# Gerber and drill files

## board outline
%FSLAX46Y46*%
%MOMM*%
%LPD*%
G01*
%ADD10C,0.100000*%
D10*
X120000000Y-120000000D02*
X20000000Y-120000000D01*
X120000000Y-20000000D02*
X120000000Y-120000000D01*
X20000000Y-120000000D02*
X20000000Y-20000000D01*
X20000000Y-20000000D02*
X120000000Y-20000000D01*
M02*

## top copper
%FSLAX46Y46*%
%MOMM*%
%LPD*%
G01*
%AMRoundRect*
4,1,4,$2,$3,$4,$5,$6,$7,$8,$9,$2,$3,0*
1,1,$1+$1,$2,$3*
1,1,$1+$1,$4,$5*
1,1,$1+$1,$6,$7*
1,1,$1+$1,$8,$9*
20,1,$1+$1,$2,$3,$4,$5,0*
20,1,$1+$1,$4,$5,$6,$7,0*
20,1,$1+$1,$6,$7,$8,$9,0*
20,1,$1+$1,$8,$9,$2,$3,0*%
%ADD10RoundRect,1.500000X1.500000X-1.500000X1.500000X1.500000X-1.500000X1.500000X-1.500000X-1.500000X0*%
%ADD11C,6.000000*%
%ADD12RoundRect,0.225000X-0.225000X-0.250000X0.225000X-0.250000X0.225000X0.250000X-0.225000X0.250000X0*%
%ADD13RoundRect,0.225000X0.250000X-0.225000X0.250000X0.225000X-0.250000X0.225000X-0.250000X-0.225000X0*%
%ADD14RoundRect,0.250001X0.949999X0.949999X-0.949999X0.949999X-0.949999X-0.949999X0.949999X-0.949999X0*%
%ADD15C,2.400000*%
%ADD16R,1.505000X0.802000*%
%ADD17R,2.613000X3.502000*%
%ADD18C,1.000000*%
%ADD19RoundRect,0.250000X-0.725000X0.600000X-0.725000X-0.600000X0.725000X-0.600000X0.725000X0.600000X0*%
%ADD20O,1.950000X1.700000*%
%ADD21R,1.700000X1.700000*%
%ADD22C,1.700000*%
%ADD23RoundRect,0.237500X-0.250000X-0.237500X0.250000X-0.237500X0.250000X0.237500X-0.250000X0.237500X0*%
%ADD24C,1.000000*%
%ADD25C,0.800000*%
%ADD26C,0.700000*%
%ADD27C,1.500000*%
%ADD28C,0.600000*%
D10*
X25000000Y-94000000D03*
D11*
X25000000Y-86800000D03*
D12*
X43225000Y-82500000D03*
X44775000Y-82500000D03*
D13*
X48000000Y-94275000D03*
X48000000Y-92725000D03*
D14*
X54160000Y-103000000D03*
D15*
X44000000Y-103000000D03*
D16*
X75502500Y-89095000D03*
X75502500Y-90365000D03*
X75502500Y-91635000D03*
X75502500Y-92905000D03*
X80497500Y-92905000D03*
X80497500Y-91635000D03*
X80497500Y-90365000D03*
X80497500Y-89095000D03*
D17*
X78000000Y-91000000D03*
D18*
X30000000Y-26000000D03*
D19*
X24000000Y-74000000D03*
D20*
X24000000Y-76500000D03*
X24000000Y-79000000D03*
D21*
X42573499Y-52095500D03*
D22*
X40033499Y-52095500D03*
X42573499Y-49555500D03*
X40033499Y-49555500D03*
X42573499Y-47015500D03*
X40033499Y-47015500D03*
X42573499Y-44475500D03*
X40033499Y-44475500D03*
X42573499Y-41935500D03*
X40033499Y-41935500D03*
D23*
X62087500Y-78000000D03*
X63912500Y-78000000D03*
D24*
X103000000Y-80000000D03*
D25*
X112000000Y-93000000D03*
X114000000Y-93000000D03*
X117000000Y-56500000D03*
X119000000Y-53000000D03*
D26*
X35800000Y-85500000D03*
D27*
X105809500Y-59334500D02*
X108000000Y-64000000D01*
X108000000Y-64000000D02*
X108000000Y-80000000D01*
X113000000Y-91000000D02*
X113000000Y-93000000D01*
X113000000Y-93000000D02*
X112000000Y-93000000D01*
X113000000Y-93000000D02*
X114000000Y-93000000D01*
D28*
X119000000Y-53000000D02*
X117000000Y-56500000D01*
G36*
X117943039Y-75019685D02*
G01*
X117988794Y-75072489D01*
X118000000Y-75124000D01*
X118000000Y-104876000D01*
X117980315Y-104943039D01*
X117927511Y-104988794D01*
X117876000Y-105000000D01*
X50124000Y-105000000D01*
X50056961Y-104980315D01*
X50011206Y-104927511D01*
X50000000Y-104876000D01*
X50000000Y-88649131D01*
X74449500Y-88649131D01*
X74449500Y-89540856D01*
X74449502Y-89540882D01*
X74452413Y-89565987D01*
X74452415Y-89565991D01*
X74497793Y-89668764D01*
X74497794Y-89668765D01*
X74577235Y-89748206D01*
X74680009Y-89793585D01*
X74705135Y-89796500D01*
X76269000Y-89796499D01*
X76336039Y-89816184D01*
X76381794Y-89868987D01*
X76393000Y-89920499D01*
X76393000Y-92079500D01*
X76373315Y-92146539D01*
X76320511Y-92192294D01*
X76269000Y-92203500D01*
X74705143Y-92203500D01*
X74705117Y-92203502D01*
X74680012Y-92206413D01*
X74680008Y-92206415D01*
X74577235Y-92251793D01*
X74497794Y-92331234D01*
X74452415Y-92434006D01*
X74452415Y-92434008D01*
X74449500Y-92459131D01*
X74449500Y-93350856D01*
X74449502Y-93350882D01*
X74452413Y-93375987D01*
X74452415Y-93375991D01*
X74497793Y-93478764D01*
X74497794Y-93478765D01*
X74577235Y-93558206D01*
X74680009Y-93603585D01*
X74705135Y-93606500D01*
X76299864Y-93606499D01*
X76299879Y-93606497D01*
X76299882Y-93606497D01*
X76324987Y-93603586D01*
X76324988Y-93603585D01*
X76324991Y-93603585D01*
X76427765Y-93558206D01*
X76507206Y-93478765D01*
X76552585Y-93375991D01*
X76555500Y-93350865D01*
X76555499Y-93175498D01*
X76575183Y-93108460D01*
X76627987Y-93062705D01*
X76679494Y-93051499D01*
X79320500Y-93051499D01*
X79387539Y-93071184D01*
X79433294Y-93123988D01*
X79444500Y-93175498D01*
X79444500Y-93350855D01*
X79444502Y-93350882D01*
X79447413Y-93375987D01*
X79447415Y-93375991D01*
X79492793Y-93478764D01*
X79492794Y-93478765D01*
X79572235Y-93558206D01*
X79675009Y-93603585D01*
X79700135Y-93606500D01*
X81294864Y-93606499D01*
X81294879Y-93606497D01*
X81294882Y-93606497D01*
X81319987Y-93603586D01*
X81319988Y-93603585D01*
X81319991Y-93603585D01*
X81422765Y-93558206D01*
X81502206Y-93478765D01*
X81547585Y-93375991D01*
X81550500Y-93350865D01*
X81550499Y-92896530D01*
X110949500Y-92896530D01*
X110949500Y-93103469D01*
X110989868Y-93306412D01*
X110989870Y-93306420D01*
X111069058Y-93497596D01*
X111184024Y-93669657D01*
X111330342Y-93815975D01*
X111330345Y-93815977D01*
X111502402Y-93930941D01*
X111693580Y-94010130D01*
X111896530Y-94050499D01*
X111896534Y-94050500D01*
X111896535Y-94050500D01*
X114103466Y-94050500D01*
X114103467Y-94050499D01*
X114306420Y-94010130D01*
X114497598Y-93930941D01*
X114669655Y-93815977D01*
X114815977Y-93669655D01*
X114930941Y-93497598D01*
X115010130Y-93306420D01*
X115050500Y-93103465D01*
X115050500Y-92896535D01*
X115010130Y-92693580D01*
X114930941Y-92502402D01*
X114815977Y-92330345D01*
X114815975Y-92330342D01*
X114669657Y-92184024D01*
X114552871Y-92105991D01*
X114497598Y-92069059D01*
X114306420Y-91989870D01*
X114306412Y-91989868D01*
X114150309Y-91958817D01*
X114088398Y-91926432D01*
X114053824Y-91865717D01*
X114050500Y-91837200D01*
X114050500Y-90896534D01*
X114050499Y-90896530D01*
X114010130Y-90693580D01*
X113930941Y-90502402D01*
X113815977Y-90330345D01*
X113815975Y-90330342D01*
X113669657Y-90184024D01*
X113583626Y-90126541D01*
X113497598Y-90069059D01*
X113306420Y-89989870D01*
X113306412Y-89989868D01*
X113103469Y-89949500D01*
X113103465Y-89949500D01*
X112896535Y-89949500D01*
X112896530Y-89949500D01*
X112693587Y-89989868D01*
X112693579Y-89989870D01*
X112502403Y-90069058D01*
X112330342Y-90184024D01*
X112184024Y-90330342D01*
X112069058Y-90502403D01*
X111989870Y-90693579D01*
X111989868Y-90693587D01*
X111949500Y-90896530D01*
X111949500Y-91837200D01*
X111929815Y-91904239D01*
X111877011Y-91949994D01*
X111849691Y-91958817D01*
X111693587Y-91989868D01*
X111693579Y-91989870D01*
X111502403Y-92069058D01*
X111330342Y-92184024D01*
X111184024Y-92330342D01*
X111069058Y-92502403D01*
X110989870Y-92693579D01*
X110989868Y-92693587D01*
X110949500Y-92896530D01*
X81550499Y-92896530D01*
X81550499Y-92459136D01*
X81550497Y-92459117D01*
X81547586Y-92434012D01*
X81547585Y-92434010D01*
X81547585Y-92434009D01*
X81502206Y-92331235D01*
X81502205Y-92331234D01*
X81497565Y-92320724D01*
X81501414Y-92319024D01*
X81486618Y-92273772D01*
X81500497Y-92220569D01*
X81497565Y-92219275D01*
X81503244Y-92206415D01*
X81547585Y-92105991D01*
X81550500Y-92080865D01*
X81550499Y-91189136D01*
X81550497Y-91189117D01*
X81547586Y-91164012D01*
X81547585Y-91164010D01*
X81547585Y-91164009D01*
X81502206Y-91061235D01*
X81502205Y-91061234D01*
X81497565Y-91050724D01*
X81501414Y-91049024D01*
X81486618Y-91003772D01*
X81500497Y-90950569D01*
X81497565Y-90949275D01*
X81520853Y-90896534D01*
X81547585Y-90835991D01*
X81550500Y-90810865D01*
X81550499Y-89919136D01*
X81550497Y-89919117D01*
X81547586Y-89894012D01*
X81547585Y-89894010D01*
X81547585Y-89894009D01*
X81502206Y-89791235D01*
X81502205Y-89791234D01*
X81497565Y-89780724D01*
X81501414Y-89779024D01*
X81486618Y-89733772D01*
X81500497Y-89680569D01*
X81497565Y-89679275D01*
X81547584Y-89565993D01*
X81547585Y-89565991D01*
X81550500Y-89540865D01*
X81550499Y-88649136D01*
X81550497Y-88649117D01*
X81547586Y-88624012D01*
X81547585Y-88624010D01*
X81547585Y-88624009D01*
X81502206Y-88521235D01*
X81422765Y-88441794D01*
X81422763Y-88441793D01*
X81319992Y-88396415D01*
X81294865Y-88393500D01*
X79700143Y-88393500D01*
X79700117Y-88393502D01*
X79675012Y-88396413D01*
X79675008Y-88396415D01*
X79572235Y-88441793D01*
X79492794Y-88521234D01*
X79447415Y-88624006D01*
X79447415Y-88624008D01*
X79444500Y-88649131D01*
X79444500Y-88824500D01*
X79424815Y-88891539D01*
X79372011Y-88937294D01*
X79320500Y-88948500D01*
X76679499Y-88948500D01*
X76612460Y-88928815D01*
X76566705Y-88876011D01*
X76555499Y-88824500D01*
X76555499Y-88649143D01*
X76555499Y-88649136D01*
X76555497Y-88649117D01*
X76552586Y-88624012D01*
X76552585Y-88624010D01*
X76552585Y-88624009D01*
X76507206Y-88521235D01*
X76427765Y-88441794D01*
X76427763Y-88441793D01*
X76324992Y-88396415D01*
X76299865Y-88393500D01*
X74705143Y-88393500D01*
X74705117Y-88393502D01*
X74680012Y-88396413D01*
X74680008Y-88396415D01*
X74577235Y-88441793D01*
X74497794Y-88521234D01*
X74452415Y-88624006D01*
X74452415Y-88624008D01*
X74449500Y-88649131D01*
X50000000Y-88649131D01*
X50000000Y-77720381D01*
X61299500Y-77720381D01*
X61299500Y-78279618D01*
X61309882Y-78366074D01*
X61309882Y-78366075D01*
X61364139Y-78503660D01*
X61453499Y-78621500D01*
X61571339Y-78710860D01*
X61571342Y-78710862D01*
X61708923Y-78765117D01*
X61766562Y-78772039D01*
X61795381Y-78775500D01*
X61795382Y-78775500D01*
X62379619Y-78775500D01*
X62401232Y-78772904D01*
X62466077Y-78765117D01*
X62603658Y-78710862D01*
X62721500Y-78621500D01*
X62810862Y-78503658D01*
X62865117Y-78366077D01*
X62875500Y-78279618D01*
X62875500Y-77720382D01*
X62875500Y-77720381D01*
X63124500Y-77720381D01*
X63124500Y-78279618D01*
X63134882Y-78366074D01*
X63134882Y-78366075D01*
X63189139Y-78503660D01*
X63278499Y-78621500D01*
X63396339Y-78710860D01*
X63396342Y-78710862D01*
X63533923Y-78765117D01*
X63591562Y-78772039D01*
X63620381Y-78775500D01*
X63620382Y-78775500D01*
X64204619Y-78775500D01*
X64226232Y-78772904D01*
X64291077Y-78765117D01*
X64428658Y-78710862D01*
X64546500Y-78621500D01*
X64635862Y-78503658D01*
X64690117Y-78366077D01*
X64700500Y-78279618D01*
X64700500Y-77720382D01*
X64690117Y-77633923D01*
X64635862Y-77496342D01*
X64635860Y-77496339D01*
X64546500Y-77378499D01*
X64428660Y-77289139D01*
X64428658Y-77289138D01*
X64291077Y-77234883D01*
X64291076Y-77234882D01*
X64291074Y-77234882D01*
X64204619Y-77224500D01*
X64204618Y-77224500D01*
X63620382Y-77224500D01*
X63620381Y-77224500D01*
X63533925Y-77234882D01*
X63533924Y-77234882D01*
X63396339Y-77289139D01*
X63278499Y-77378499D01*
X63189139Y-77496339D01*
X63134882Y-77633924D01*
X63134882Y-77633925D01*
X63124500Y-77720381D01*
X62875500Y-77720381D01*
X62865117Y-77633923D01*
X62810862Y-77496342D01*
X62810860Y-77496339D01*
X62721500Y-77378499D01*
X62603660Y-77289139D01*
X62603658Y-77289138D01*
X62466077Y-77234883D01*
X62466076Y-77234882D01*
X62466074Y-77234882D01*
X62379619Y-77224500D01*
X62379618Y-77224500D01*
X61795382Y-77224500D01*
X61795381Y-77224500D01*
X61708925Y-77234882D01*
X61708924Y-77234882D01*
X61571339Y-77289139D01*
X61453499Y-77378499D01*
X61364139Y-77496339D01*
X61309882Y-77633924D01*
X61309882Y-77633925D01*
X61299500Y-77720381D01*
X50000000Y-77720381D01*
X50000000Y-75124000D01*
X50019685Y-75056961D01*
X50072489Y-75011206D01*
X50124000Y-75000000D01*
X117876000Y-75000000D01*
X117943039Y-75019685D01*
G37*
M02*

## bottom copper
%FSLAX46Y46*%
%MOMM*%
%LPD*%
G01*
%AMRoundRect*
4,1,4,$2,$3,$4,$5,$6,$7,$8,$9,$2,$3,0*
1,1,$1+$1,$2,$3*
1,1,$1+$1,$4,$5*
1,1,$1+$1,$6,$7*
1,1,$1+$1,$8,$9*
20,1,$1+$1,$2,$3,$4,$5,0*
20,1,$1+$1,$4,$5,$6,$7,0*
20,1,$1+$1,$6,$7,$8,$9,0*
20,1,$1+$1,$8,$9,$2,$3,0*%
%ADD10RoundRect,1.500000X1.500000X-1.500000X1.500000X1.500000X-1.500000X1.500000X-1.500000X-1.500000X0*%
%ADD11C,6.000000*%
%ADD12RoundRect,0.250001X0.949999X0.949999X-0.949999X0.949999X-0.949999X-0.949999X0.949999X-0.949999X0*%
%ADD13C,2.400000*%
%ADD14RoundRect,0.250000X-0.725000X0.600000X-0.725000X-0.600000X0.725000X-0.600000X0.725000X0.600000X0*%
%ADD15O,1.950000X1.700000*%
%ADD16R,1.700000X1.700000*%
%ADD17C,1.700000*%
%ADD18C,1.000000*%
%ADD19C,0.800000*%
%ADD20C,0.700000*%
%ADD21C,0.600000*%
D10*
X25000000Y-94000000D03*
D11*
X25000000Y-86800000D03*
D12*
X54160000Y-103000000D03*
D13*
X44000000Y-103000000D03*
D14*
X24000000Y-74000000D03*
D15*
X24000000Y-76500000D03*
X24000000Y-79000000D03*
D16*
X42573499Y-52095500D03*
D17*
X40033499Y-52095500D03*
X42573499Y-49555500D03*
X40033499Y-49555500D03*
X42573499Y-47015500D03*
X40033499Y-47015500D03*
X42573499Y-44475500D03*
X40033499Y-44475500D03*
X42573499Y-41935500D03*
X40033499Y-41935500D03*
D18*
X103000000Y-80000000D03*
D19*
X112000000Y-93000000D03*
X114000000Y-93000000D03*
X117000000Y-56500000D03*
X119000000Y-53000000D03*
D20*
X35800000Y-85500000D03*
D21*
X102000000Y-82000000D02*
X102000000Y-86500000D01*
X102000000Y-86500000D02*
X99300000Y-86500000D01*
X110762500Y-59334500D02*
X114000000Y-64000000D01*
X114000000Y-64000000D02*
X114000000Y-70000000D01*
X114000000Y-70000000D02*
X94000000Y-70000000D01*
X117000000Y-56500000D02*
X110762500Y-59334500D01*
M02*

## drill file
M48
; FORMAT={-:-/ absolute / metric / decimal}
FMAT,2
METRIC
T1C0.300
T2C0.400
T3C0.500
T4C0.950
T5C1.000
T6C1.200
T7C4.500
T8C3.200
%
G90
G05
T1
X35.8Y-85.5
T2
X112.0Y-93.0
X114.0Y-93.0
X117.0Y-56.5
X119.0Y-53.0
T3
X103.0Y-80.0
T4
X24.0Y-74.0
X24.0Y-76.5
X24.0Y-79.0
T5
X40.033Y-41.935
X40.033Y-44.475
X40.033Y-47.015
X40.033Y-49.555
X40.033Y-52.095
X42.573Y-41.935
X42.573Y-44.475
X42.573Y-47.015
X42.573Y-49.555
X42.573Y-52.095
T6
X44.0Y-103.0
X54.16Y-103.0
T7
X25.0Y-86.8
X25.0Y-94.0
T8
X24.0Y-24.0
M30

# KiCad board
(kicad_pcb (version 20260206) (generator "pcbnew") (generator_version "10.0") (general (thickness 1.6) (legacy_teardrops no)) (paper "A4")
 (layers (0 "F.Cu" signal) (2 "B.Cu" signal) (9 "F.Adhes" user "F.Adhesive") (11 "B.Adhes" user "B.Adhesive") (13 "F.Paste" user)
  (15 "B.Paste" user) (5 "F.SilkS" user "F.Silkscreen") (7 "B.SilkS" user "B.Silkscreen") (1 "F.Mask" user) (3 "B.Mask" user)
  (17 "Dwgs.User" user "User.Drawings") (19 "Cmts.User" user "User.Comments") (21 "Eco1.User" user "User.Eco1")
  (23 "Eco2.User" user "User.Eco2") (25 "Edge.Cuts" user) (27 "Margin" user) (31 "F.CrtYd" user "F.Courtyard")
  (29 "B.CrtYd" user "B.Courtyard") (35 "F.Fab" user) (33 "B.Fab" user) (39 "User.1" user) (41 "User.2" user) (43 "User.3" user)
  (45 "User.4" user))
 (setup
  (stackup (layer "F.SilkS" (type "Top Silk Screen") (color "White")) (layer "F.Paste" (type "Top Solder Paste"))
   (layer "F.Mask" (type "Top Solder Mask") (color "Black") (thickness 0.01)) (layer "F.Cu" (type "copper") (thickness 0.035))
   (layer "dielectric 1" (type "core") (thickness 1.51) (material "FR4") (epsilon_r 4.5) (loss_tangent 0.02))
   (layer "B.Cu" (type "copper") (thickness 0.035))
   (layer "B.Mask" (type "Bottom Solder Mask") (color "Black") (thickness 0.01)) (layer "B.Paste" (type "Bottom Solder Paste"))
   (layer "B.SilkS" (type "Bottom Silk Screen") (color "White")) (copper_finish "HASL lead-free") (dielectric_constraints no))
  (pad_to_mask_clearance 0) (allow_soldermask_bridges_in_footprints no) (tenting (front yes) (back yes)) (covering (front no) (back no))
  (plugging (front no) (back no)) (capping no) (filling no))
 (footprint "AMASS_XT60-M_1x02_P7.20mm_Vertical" (layer "F.Cu") (at 25 94 90)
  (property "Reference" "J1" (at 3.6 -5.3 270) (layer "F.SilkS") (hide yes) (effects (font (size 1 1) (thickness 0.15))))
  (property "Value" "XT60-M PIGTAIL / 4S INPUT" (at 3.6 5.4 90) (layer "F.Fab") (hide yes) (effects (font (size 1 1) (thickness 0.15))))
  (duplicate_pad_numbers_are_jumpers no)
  (pad "1" thru_hole roundrect (at 0 0 90) (size 6 6) (drill 4.5) (layers "*.Cu" "*.Mask") (remove_unused_layers no) (roundrect_rratio 0.25)
   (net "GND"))
  (pad "2" thru_hole circle (at 7.2 0 90) (size 6 6) (drill 4.5) (layers "*.Cu" "*.Mask") (remove_unused_layers no) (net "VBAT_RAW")))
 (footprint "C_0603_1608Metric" (layer "F.Cu") (at 44 82.5)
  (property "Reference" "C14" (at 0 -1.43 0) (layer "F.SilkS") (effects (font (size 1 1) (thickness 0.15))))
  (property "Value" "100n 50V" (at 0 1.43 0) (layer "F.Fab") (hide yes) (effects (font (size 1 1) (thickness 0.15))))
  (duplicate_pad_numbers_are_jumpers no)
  (pad "1" smd roundrect (at -0.775 0) (size 0.9 0.95) (layers "F.Cu" "F.Mask" "F.Paste") (roundrect_rratio 0.25) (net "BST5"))
  (pad "2" smd roundrect (at 0.775 0) (size 0.9 0.95) (layers "F.Cu" "F.Mask" "F.Paste") (roundrect_rratio 0.25) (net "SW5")))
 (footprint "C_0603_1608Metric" (layer "F.Cu") (at 48 93.5 90)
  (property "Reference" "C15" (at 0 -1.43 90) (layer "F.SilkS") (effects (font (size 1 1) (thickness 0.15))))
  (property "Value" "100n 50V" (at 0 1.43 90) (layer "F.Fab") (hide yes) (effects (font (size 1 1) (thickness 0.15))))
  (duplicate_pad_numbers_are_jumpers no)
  (pad "1" smd roundrect (at -0.775 0 90) (size 0.9 0.95) (layers "F.Cu" "F.Mask" "F.Paste") (roundrect_rratio 0.25) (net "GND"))
  (pad "2" smd roundrect (at 0.775 0 90) (size 0.9 0.95) (layers "F.Cu" "F.Mask" "F.Paste") (roundrect_rratio 0.25) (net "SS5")))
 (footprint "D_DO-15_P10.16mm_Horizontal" (layer "F.Cu") (at 54.16 103 180)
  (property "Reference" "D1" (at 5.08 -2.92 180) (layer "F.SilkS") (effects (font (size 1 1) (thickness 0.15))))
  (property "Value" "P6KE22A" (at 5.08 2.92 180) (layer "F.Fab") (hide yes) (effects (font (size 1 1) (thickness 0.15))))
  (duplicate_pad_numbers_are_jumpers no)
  (pad "1" thru_hole roundrect (at 0 0 180) (size 2.4 2.4) (drill 1.2) (layers "*.Cu" "*.Mask") (remove_unused_layers no)
   (roundrect_rratio 0.104167) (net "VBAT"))
  (pad "2" thru_hole circle (at 10.16 0 180) (size 2.4 2.4) (drill 1.2) (layers "*.Cu" "*.Mask") (remove_unused_layers no) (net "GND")))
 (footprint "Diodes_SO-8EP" (layer "F.Cu") (at 78 91)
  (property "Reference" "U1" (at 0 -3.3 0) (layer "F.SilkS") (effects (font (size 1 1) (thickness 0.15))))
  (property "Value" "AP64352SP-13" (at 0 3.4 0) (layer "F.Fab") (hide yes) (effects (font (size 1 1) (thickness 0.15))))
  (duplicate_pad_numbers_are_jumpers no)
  (pad "1" smd rect (at -2.4975 -1.905) (size 1.505 0.802) (layers "F.Cu" "F.Mask" "F.Paste") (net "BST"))
  (pad "2" smd rect (at -2.4975 -0.635) (size 1.505 0.802) (layers "F.Cu" "F.Mask" "F.Paste") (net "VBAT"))
  (pad "3" smd rect (at -2.4975 0.635) (size 1.505 0.802) (layers "F.Cu" "F.Mask" "F.Paste") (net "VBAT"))
  (pad "4" smd rect (at -2.4975 1.905) (size 1.505 0.802) (layers "F.Cu" "F.Mask" "F.Paste") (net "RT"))
  (pad "5" smd rect (at 2.4975 1.905) (size 1.505 0.802) (layers "F.Cu" "F.Mask" "F.Paste") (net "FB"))
  (pad "6" smd rect (at 2.4975 0.635) (size 1.505 0.802) (layers "F.Cu" "F.Mask" "F.Paste") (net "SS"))
  (pad "7" smd rect (at 2.4975 -0.635) (size 1.505 0.802) (layers "F.Cu" "F.Mask" "F.Paste") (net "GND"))
  (pad "8" smd rect (at 2.4975 -1.905) (size 1.505 0.802) (layers "F.Cu" "F.Mask" "F.Paste") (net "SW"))
  (pad "9" smd rect (at 0 0) (size 2.613 3.502) (layers "F.Cu" "F.Mask" "F.Paste") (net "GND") (solder_paste_margin_ratio -0.2)))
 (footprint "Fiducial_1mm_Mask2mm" (layer "F.Cu") (at 30 26)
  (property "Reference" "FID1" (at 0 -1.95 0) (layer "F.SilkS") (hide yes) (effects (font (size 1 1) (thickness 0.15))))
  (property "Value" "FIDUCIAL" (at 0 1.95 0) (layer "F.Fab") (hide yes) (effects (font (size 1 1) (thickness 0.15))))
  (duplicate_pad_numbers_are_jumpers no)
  (pad "" smd circle (at 0 0) (size 1 1) (layers "F.Cu" "F.Mask") (solder_mask_margin 0.5) (clearance 0.6)))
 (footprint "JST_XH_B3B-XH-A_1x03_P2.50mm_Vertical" (layer "F.Cu") (at 24 74 -90)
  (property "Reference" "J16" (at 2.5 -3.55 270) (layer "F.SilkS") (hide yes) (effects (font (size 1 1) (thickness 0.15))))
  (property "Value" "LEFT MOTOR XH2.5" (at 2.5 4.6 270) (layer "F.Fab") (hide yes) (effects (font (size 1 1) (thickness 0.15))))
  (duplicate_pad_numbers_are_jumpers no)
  (pad "1" thru_hole roundrect (at 0 0 270) (size 1.7 1.95) (drill 0.95) (layers "*.Cu" "*.Mask") (remove_unused_layers no)
   (roundrect_rratio 0.147059) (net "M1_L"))
  (pad "2" thru_hole oval (at 2.5 0 270) (size 1.7 1.95) (drill 0.95) (layers "*.Cu" "*.Mask") (remove_unused_layers no) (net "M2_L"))
  (pad "3" thru_hole oval (at 5 0 270) (size 1.7 1.95) (drill 0.95) (layers "*.Cu" "*.Mask") (remove_unused_layers no) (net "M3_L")))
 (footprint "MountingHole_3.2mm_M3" (layer "F.Cu") (at 24 24)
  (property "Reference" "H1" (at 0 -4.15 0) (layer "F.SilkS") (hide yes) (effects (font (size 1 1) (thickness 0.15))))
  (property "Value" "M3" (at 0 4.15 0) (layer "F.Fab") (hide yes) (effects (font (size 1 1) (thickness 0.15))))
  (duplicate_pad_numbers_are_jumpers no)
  (pad "" np_thru_hole circle (at 0 0) (size 3.2 3.2) (drill 3.2) (layers "*.Cu" "*.Mask")))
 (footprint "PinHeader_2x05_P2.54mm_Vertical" (layer "F.Cu") (at 42.573499 52.0955 180)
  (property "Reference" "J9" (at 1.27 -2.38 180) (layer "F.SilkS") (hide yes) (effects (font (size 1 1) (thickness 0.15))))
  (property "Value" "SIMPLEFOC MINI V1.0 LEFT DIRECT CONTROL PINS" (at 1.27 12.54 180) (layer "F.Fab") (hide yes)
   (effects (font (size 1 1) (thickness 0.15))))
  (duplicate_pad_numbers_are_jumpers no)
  (pad "1" thru_hole rect (at 0 0 180) (size 1.7 1.7) (drill 1) (layers "*.Cu" "*.Mask") (remove_unused_layers no) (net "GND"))
  (pad "2" thru_hole circle (at 2.54 0 180) (size 1.7 1.7) (drill 1) (layers "*.Cu" "*.Mask") (remove_unused_layers no))
  (pad "3" thru_hole circle (at 0 2.54 180) (size 1.7 1.7) (drill 1) (layers "*.Cu" "*.Mask") (remove_unused_layers no) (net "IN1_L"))
  (pad "4" thru_hole circle (at 2.54 2.54 180) (size 1.7 1.7) (drill 1) (layers "*.Cu" "*.Mask") (remove_unused_layers no) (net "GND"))
  (pad "5" thru_hole circle (at 0 5.08 180) (size 1.7 1.7) (drill 1) (layers "*.Cu" "*.Mask") (remove_unused_layers no) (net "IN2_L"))
  (pad "6" thru_hole circle (at 2.54 5.08 180) (size 1.7 1.7) (drill 1) (layers "*.Cu" "*.Mask") (remove_unused_layers no))
  (pad "7" thru_hole circle (at 0 7.62 180) (size 1.7 1.7) (drill 1) (layers "*.Cu" "*.Mask") (remove_unused_layers no) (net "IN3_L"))
  (pad "8" thru_hole circle (at 2.54 7.62 180) (size 1.7 1.7) (drill 1) (layers "*.Cu" "*.Mask") (remove_unused_layers no))
  (pad "9" thru_hole circle (at 0 10.16 180) (size 1.7 1.7) (drill 1) (layers "*.Cu" "*.Mask") (remove_unused_layers no) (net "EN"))
  (pad "10" thru_hole circle (at 2.54 10.16 180) (size 1.7 1.7) (drill 1) (layers "*.Cu" "*.Mask") (remove_unused_layers no)
   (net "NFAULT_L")))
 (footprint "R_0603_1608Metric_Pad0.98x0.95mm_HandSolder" (layer "F.Cu") (at 63 78)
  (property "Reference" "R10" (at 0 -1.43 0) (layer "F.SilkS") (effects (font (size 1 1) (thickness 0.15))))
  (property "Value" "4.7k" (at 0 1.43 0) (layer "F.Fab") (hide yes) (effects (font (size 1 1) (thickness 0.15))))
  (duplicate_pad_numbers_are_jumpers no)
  (pad "1" smd roundrect (at -0.9125 0) (size 0.975 0.95) (layers "F.Cu" "F.Mask" "F.Paste") (roundrect_rratio 0.25) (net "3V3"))
  (pad "2" smd roundrect (at 0.9125 0) (size 0.975 0.95) (layers "F.Cu" "F.Mask" "F.Paste") (roundrect_rratio 0.25) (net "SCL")))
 (gr_line (start 120 120) (end 20 120) (stroke (width 0.1) (type default)) (layer "Edge.Cuts"))
 (gr_line (start 120 20) (end 120 120) (stroke (width 0.1) (type default)) (layer "Edge.Cuts"))
 (gr_line (start 20 120) (end 20 20) (stroke (width 0.1) (type default)) (layer "Edge.Cuts"))
 (gr_line (start 20 20) (end 120 20) (stroke (width 0.1) (type default)) (layer "Edge.Cuts"))
 (segment (start 102 82) (end 102 86.5) (width 0.6) (layer "B.Cu") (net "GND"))
 (segment (start 102 86.5) (end 99.3 86.5) (width 0.6) (layer "B.Cu") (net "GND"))
 (segment (start 105.8095 59.3345) (end 108 64) (width 1.5) (layer "F.Cu") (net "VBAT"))
 (segment (start 108 64) (end 108 80) (width 1.5) (layer "F.Cu") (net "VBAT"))
 (segment (start 110.7625 59.3345) (end 114 64) (width 0.6) (layer "B.Cu") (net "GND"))
 (segment (start 113 91) (end 113 93) (width 1.5) (layer "F.Cu") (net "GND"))
 (segment (start 113 93) (end 112 93) (width 1.5) (layer "F.Cu") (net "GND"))
 (segment (start 113 93) (end 114 93) (width 1.5) (layer "F.Cu") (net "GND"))
 (segment (start 114 64) (end 114 70) (width 0.6) (layer "B.Cu") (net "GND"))
 (segment (start 114 70) (end 94 70) (width 0.6) (layer "B.Cu") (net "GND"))
 (segment (start 117 56.5) (end 110.7625 59.3345) (width 0.6) (layer "B.Cu") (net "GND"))
 (segment (start 119 53) (end 117 56.5) (width 0.6) (layer "F.Cu") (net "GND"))
 (via (at 103 80) (size 1) (drill 0.5) (layers "F.Cu" "B.Cu") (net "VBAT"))
 (via (at 112 93) (size 0.8) (drill 0.4) (layers "F.Cu" "B.Cu") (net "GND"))
 (via (at 114 93) (size 0.8) (drill 0.4) (layers "F.Cu" "B.Cu") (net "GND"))
 (via (at 117 56.5) (size 0.8) (drill 0.4) (layers "F.Cu" "B.Cu") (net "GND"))
 (via (at 119 53) (size 0.8) (drill 0.4) (layers "F.Cu" "B.Cu") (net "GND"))
 (via (at 35.8 85.5) (size 0.7) (drill 0.3) (layers "F.Cu" "B.Cu") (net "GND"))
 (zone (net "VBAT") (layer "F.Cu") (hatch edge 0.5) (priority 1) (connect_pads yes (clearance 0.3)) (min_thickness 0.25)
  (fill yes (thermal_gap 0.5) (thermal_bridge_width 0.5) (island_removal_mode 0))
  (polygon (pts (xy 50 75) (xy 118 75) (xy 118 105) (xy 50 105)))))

